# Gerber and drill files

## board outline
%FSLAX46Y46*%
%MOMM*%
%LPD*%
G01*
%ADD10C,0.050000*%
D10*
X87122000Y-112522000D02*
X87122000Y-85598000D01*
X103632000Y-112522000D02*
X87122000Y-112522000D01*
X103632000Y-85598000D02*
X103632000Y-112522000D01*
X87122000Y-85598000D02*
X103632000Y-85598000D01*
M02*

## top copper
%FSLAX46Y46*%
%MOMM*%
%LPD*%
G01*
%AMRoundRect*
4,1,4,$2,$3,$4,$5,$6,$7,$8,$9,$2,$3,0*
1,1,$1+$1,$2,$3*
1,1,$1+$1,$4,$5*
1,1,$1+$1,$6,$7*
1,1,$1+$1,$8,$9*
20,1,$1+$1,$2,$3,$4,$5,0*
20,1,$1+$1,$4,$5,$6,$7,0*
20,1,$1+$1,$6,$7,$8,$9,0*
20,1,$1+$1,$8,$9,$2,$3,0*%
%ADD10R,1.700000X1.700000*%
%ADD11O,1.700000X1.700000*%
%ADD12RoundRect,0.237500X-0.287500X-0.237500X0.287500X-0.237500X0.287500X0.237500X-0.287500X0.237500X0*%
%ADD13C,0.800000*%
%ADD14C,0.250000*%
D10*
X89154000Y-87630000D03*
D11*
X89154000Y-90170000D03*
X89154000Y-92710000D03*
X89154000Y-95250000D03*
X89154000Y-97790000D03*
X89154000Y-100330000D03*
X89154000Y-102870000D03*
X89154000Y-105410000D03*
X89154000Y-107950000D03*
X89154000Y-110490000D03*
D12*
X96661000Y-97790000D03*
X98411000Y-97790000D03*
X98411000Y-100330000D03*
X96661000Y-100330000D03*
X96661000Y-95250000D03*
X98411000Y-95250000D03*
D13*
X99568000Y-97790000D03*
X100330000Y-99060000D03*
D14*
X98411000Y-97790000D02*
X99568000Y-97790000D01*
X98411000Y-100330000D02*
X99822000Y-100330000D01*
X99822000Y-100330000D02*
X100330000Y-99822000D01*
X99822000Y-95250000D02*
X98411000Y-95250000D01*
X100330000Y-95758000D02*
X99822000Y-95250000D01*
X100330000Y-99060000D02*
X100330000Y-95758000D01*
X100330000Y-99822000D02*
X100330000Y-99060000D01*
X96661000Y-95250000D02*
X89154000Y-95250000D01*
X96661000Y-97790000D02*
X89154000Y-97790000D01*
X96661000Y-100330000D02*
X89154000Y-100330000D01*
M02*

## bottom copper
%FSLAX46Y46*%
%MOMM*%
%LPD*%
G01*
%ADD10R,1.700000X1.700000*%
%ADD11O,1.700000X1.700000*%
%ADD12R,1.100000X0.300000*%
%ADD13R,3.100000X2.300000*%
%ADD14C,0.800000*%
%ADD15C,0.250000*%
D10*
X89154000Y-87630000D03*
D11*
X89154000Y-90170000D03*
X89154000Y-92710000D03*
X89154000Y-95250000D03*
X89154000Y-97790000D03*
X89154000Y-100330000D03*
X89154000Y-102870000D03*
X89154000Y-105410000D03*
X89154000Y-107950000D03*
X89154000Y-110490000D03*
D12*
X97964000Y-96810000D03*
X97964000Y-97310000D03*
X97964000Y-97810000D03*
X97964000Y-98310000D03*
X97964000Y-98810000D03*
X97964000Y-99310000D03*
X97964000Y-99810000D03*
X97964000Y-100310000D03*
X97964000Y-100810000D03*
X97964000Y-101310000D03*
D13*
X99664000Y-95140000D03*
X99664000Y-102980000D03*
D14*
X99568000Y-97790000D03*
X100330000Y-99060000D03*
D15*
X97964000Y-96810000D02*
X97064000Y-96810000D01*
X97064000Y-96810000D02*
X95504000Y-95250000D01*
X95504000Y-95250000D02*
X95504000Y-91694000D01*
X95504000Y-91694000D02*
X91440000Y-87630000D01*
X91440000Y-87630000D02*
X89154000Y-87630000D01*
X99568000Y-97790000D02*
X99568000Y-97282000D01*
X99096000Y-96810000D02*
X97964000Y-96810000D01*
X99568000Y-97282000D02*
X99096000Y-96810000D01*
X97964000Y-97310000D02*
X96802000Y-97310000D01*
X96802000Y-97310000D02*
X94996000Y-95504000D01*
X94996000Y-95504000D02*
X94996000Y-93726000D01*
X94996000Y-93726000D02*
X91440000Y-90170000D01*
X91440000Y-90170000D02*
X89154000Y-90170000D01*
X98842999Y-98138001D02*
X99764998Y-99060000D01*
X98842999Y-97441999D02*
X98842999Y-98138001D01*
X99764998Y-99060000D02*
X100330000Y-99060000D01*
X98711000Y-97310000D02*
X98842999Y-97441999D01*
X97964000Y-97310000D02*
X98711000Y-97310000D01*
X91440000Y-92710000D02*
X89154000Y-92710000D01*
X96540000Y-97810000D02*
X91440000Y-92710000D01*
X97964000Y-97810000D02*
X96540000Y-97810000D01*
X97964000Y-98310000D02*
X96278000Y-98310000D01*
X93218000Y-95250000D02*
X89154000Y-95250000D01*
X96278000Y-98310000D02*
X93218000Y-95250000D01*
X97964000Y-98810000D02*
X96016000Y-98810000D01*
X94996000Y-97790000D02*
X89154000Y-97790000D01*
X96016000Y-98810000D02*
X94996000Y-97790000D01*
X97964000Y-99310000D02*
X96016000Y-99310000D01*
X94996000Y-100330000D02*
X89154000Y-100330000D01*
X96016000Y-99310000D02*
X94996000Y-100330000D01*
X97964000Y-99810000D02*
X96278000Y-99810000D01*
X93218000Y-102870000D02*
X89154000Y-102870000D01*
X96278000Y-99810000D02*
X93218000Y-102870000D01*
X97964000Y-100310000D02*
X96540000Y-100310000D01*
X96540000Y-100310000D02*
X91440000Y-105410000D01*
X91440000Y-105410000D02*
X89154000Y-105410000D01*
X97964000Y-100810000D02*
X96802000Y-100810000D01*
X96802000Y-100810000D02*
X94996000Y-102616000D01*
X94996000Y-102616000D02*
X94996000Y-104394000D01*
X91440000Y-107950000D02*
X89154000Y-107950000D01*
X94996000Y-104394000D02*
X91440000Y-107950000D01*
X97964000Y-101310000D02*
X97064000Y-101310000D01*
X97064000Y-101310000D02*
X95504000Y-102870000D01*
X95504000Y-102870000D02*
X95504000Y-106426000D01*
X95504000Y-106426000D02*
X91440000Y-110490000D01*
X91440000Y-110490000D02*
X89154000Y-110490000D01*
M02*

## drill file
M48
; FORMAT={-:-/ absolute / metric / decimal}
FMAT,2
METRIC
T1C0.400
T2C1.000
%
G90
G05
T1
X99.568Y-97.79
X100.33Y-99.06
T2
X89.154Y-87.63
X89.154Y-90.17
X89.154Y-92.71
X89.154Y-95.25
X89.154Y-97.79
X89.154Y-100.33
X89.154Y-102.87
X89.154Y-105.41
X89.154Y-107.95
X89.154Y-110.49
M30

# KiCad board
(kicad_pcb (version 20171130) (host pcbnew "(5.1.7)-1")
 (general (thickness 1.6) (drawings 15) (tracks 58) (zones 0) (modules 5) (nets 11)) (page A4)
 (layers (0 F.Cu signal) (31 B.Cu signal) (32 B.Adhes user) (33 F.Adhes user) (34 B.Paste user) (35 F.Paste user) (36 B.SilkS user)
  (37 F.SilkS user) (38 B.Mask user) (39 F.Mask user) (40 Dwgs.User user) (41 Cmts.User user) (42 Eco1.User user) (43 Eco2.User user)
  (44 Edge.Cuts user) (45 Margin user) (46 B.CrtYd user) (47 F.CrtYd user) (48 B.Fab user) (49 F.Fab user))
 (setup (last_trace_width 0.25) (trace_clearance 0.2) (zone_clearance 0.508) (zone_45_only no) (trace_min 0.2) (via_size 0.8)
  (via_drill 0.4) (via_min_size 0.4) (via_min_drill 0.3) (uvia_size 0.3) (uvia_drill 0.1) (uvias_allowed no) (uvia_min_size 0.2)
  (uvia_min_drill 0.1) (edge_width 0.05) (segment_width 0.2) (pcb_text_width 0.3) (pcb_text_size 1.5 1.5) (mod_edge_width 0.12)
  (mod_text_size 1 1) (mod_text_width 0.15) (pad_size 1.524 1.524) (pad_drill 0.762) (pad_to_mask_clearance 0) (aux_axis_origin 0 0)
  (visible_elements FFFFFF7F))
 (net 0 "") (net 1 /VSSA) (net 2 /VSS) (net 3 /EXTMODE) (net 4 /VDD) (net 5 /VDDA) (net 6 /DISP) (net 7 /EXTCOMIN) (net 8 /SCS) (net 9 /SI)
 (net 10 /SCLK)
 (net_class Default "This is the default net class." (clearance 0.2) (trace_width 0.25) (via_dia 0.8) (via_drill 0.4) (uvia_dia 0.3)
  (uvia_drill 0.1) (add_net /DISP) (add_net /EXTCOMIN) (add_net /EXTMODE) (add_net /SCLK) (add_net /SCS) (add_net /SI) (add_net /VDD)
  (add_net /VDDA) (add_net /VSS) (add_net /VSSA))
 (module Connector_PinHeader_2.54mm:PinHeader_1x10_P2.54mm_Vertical (layer F.Cu) (at 89.154 87.63)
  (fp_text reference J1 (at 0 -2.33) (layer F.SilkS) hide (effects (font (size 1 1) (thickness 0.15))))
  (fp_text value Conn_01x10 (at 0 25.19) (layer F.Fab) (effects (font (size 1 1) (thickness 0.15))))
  (pad 1 thru_hole rect (at 0 0) (size 1.7 1.7) (drill 1) (layers *.Cu *.Mask) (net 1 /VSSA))
  (pad 2 thru_hole oval (at 0 2.54) (size 1.7 1.7) (drill 1) (layers *.Cu *.Mask) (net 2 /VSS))
  (pad 3 thru_hole oval (at 0 5.08) (size 1.7 1.7) (drill 1) (layers *.Cu *.Mask) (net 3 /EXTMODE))
  (pad 4 thru_hole oval (at 0 7.62) (size 1.7 1.7) (drill 1) (layers *.Cu *.Mask) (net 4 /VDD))
  (pad 5 thru_hole oval (at 0 10.16) (size 1.7 1.7) (drill 1) (layers *.Cu *.Mask) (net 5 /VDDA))
  (pad 6 thru_hole oval (at 0 12.7) (size 1.7 1.7) (drill 1) (layers *.Cu *.Mask) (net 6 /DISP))
  (pad 7 thru_hole oval (at 0 15.24) (size 1.7 1.7) (drill 1) (layers *.Cu *.Mask) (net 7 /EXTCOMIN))
  (pad 8 thru_hole oval (at 0 17.78) (size 1.7 1.7) (drill 1) (layers *.Cu *.Mask) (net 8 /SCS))
  (pad 9 thru_hole oval (at 0 20.32) (size 1.7 1.7) (drill 1) (layers *.Cu *.Mask) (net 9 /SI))
  (pad 10 thru_hole oval (at 0 22.86) (size 1.7 1.7) (drill 1) (layers *.Cu *.Mask) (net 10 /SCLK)))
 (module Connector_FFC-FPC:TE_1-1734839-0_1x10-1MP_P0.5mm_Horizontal (layer B.Cu) (at 99.314 99.06 270)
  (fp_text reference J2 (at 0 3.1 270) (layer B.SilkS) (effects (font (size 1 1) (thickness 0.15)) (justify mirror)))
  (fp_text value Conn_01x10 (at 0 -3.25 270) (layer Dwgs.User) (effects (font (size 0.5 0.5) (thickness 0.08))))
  (pad 1 smd rect (at -2.25 1.35 270) (size 0.3 1.1) (layers B.Cu B.Paste B.Mask) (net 1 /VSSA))
  (pad 2 smd rect (at -1.75 1.35 270) (size 0.3 1.1) (layers B.Cu B.Paste B.Mask) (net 2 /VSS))
  (pad 3 smd rect (at -1.25 1.35 270) (size 0.3 1.1) (layers B.Cu B.Paste B.Mask) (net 3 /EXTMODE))
  (pad 4 smd rect (at -0.75 1.35 270) (size 0.3 1.1) (layers B.Cu B.Paste B.Mask) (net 4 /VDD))
  (pad 5 smd rect (at -0.25 1.35 270) (size 0.3 1.1) (layers B.Cu B.Paste B.Mask) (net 5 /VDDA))
  (pad 6 smd rect (at 0.25 1.35 270) (size 0.3 1.1) (layers B.Cu B.Paste B.Mask) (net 6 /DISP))
  (pad 7 smd rect (at 0.75 1.35 270) (size 0.3 1.1) (layers B.Cu B.Paste B.Mask) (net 7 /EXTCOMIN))
  (pad 8 smd rect (at 1.25 1.35 270) (size 0.3 1.1) (layers B.Cu B.Paste B.Mask) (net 8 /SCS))
  (pad 9 smd rect (at 1.75 1.35 270) (size 0.3 1.1) (layers B.Cu B.Paste B.Mask) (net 9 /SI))
  (pad 10 smd rect (at 2.25 1.35 270) (size 0.3 1.1) (layers B.Cu B.Paste B.Mask) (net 10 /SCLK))
  (pad MP smd rect (at -3.92 -0.35 270) (size 2.3 3.1) (layers B.Cu B.Paste B.Mask))
  (pad MP smd rect (at 3.92 -0.35 270) (size 2.3 3.1) (layers B.Cu B.Paste B.Mask)))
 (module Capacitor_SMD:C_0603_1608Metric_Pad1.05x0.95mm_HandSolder (layer F.Cu) (at 97.536 97.79)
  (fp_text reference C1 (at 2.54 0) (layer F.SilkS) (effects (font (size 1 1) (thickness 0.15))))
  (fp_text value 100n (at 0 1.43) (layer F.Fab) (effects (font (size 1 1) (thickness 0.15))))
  (pad 1 smd roundrect (at -0.875 0) (size 1.05 0.95) (layers F.Cu F.Paste F.Mask) (roundrect_rratio 0.25) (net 5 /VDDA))
  (pad 2 smd roundrect (at 0.875 0) (size 1.05 0.95) (layers F.Cu F.Paste F.Mask) (roundrect_rratio 0.25) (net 1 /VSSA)))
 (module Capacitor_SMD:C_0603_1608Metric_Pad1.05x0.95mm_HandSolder (layer F.Cu) (at 97.536 100.33)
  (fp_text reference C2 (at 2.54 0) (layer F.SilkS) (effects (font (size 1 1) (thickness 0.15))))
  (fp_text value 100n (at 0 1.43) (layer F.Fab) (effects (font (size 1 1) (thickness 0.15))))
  (pad 2 smd roundrect (at 0.875 0) (size 1.05 0.95) (layers F.Cu F.Paste F.Mask) (roundrect_rratio 0.25) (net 2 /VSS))
  (pad 1 smd roundrect (at -0.875 0) (size 1.05 0.95) (layers F.Cu F.Paste F.Mask) (roundrect_rratio 0.25) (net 6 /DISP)))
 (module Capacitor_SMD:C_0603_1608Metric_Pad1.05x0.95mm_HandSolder (layer F.Cu) (at 97.536 95.25)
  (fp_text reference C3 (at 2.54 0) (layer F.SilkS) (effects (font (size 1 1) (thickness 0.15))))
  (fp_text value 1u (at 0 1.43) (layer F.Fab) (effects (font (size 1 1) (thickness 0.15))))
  (pad 1 smd roundrect (at -0.875 0) (size 1.05 0.95) (layers F.Cu F.Paste F.Mask) (roundrect_rratio 0.25) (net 4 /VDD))
  (pad 2 smd roundrect (at 0.875 0) (size 1.05 0.95) (layers F.Cu F.Paste F.Mask) (roundrect_rratio 0.25) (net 2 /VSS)))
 (gr_line (start 87.122 112.522) (end 87.122 85.598) (layer Edge.Cuts) (width 0.05))
 (gr_line (start 103.632 112.522) (end 87.122 112.522) (layer Edge.Cuts) (width 0.05))
 (gr_line (start 103.632 85.598) (end 103.632 112.522) (layer Edge.Cuts) (width 0.05))
 (gr_line (start 87.122 85.598) (end 103.632 85.598) (layer Edge.Cuts) (width 0.05))
 (segment (start 97.964 96.81) (end 97.064 96.81) (width 0.25) (layer B.Cu) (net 1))
 (segment (start 97.064 96.81) (end 95.504 95.25) (width 0.25) (layer B.Cu) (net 1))
 (segment (start 95.504 95.25) (end 95.504 91.694) (width 0.25) (layer B.Cu) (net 1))
 (segment (start 95.504 91.694) (end 91.44 87.63) (width 0.25) (layer B.Cu) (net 1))
 (segment (start 91.44 87.63) (end 89.154 87.63) (width 0.25) (layer B.Cu) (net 1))
 (via (at 99.568 97.79) (size 0.8) (drill 0.4) (layers F.Cu B.Cu) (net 1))
 (segment (start 98.411 97.79) (end 99.568 97.79) (width 0.25) (layer F.Cu) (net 1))
 (segment (start 99.568 97.79) (end 99.568 97.282) (width 0.25) (layer B.Cu) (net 1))
 (segment (start 99.096 96.81) (end 97.964 96.81) (width 0.25) (layer B.Cu) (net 1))
 (segment (start 99.568 97.282) (end 99.096 96.81) (width 0.25) (layer B.Cu) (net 1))
 (segment (start 97.964 97.31) (end 96.802 97.31) (width 0.25) (layer B.Cu) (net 2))
 (segment (start 96.802 97.31) (end 94.996 95.504) (width 0.25) (layer B.Cu) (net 2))
 (segment (start 94.996 95.504) (end 94.996 93.726) (width 0.25) (layer B.Cu) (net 2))
 (segment (start 94.996 93.726) (end 91.44 90.17) (width 0.25) (layer B.Cu) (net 2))
 (segment (start 91.44 90.17) (end 89.154 90.17) (width 0.25) (layer B.Cu) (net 2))
 (segment (start 98.411 100.33) (end 99.822 100.33) (width 0.25) (layer F.Cu) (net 2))
 (segment (start 99.822 100.33) (end 100.33 99.822) (width 0.25) (layer F.Cu) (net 2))
 (segment (start 99.822 95.25) (end 98.411 95.25) (width 0.25) (layer F.Cu) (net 2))
 (segment (start 100.33 95.758) (end 99.822 95.25) (width 0.25) (layer F.Cu) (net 2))
 (via (at 100.33 99.06) (size 0.8) (drill 0.4) (layers F.Cu B.Cu) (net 2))
 (segment (start 98.842999 98.138001) (end 99.764998 99.06) (width 0.25) (layer B.Cu) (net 2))
 (segment (start 98.842999 97.441999) (end 98.842999 98.138001) (width 0.25) (layer B.Cu) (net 2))
 (segment (start 99.764998 99.06) (end 100.33 99.06) (width 0.25) (layer B.Cu) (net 2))
 (segment (start 98.711 97.31) (end 98.842999 97.441999) (width 0.25) (layer B.Cu) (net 2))
 (segment (start 97.964 97.31) (end 98.711 97.31) (width 0.25) (layer B.Cu) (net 2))
 (segment (start 100.33 99.06) (end 100.33 95.758) (width 0.25) (layer F.Cu) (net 2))
 (segment (start 100.33 99.822) (end 100.33 99.06) (width 0.25) (layer F.Cu) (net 2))
 (segment (start 91.44 92.71) (end 89.154 92.71) (width 0.25) (layer B.Cu) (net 3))
 (segment (start 96.54 97.81) (end 91.44 92.71) (width 0.25) (layer B.Cu) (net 3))
 (segment (start 97.964 97.81) (end 96.54 97.81) (width 0.25) (layer B.Cu) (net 3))
 (segment (start 97.964 98.31) (end 96.278 98.31) (width 0.25) (layer B.Cu) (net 4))
 (segment (start 93.218 95.25) (end 89.154 95.25) (width 0.25) (layer B.Cu) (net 4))
 (segment (start 96.278 98.31) (end 93.218 95.25) (width 0.25) (layer B.Cu) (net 4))
 (segment (start 96.661 95.25) (end 89.154 95.25) (width 0.25) (layer F.Cu) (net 4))
 (segment (start 97.964 98.81) (end 96.016 98.81) (width 0.25) (layer B.Cu) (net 5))
 (segment (start 94.996 97.79) (end 89.154 97.79) (width 0.25) (layer B.Cu) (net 5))
 (segment (start 96.016 98.81) (end 94.996 97.79) (width 0.25) (layer B.Cu) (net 5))
 (segment (start 96.661 97.79) (end 89.154 97.79) (width 0.25) (layer F.Cu) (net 5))
 (segment (start 97.964 99.31) (end 96.016 99.31) (width 0.25) (layer B.Cu) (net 6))
 (segment (start 94.996 100.33) (end 89.154 100.33) (width 0.25) (layer B.Cu) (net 6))
 (segment (start 96.016 99.31) (end 94.996 100.33) (width 0.25) (layer B.Cu) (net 6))
 (segment (start 96.661 100.33) (end 89.154 100.33) (width 0.25) (layer F.Cu) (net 6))
 (segment (start 97.964 99.81) (end 96.278 99.81) (width 0.25) (layer B.Cu) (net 7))
 (segment (start 93.218 102.87) (end 89.154 102.87) (width 0.25) (layer B.Cu) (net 7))
 (segment (start 96.278 99.81) (end 93.218 102.87) (width 0.25) (layer B.Cu) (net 7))
 (segment (start 97.964 100.31) (end 96.54 100.31) (width 0.25) (layer B.Cu) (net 8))
 (segment (start 96.54 100.31) (end 91.44 105.41) (width 0.25) (layer B.Cu) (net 8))
 (segment (start 91.44 105.41) (end 89.154 105.41) (width 0.25) (layer B.Cu) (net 8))
 (segment (start 97.964 100.81) (end 96.802 100.81) (width 0.25) (layer B.Cu) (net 9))
 (segment (start 96.802 100.81) (end 94.996 102.616) (width 0.25) (layer B.Cu) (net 9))
 (segment (start 94.996 102.616) (end 94.996 104.394) (width 0.25) (layer B.Cu) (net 9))
 (segment (start 91.44 107.95) (end 89.154 107.95) (width 0.25) (layer B.Cu) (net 9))
 (segment (start 94.996 104.394) (end 91.44 107.95) (width 0.25) (layer B.Cu) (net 9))
 (segment (start 97.964 101.31) (end 97.064 101.31) (width 0.25) (layer B.Cu) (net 10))
 (segment (start 97.064 101.31) (end 95.504 102.87) (width 0.25) (layer B.Cu) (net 10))
 (segment (start 95.504 102.87) (end 95.504 106.426) (width 0.25) (layer B.Cu) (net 10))
 (segment (start 95.504 106.426) (end 91.44 110.49) (width 0.25) (layer B.Cu) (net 10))
 (segment (start 91.44 110.49) (end 89.154 110.49) (width 0.25) (layer B.Cu) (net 10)))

